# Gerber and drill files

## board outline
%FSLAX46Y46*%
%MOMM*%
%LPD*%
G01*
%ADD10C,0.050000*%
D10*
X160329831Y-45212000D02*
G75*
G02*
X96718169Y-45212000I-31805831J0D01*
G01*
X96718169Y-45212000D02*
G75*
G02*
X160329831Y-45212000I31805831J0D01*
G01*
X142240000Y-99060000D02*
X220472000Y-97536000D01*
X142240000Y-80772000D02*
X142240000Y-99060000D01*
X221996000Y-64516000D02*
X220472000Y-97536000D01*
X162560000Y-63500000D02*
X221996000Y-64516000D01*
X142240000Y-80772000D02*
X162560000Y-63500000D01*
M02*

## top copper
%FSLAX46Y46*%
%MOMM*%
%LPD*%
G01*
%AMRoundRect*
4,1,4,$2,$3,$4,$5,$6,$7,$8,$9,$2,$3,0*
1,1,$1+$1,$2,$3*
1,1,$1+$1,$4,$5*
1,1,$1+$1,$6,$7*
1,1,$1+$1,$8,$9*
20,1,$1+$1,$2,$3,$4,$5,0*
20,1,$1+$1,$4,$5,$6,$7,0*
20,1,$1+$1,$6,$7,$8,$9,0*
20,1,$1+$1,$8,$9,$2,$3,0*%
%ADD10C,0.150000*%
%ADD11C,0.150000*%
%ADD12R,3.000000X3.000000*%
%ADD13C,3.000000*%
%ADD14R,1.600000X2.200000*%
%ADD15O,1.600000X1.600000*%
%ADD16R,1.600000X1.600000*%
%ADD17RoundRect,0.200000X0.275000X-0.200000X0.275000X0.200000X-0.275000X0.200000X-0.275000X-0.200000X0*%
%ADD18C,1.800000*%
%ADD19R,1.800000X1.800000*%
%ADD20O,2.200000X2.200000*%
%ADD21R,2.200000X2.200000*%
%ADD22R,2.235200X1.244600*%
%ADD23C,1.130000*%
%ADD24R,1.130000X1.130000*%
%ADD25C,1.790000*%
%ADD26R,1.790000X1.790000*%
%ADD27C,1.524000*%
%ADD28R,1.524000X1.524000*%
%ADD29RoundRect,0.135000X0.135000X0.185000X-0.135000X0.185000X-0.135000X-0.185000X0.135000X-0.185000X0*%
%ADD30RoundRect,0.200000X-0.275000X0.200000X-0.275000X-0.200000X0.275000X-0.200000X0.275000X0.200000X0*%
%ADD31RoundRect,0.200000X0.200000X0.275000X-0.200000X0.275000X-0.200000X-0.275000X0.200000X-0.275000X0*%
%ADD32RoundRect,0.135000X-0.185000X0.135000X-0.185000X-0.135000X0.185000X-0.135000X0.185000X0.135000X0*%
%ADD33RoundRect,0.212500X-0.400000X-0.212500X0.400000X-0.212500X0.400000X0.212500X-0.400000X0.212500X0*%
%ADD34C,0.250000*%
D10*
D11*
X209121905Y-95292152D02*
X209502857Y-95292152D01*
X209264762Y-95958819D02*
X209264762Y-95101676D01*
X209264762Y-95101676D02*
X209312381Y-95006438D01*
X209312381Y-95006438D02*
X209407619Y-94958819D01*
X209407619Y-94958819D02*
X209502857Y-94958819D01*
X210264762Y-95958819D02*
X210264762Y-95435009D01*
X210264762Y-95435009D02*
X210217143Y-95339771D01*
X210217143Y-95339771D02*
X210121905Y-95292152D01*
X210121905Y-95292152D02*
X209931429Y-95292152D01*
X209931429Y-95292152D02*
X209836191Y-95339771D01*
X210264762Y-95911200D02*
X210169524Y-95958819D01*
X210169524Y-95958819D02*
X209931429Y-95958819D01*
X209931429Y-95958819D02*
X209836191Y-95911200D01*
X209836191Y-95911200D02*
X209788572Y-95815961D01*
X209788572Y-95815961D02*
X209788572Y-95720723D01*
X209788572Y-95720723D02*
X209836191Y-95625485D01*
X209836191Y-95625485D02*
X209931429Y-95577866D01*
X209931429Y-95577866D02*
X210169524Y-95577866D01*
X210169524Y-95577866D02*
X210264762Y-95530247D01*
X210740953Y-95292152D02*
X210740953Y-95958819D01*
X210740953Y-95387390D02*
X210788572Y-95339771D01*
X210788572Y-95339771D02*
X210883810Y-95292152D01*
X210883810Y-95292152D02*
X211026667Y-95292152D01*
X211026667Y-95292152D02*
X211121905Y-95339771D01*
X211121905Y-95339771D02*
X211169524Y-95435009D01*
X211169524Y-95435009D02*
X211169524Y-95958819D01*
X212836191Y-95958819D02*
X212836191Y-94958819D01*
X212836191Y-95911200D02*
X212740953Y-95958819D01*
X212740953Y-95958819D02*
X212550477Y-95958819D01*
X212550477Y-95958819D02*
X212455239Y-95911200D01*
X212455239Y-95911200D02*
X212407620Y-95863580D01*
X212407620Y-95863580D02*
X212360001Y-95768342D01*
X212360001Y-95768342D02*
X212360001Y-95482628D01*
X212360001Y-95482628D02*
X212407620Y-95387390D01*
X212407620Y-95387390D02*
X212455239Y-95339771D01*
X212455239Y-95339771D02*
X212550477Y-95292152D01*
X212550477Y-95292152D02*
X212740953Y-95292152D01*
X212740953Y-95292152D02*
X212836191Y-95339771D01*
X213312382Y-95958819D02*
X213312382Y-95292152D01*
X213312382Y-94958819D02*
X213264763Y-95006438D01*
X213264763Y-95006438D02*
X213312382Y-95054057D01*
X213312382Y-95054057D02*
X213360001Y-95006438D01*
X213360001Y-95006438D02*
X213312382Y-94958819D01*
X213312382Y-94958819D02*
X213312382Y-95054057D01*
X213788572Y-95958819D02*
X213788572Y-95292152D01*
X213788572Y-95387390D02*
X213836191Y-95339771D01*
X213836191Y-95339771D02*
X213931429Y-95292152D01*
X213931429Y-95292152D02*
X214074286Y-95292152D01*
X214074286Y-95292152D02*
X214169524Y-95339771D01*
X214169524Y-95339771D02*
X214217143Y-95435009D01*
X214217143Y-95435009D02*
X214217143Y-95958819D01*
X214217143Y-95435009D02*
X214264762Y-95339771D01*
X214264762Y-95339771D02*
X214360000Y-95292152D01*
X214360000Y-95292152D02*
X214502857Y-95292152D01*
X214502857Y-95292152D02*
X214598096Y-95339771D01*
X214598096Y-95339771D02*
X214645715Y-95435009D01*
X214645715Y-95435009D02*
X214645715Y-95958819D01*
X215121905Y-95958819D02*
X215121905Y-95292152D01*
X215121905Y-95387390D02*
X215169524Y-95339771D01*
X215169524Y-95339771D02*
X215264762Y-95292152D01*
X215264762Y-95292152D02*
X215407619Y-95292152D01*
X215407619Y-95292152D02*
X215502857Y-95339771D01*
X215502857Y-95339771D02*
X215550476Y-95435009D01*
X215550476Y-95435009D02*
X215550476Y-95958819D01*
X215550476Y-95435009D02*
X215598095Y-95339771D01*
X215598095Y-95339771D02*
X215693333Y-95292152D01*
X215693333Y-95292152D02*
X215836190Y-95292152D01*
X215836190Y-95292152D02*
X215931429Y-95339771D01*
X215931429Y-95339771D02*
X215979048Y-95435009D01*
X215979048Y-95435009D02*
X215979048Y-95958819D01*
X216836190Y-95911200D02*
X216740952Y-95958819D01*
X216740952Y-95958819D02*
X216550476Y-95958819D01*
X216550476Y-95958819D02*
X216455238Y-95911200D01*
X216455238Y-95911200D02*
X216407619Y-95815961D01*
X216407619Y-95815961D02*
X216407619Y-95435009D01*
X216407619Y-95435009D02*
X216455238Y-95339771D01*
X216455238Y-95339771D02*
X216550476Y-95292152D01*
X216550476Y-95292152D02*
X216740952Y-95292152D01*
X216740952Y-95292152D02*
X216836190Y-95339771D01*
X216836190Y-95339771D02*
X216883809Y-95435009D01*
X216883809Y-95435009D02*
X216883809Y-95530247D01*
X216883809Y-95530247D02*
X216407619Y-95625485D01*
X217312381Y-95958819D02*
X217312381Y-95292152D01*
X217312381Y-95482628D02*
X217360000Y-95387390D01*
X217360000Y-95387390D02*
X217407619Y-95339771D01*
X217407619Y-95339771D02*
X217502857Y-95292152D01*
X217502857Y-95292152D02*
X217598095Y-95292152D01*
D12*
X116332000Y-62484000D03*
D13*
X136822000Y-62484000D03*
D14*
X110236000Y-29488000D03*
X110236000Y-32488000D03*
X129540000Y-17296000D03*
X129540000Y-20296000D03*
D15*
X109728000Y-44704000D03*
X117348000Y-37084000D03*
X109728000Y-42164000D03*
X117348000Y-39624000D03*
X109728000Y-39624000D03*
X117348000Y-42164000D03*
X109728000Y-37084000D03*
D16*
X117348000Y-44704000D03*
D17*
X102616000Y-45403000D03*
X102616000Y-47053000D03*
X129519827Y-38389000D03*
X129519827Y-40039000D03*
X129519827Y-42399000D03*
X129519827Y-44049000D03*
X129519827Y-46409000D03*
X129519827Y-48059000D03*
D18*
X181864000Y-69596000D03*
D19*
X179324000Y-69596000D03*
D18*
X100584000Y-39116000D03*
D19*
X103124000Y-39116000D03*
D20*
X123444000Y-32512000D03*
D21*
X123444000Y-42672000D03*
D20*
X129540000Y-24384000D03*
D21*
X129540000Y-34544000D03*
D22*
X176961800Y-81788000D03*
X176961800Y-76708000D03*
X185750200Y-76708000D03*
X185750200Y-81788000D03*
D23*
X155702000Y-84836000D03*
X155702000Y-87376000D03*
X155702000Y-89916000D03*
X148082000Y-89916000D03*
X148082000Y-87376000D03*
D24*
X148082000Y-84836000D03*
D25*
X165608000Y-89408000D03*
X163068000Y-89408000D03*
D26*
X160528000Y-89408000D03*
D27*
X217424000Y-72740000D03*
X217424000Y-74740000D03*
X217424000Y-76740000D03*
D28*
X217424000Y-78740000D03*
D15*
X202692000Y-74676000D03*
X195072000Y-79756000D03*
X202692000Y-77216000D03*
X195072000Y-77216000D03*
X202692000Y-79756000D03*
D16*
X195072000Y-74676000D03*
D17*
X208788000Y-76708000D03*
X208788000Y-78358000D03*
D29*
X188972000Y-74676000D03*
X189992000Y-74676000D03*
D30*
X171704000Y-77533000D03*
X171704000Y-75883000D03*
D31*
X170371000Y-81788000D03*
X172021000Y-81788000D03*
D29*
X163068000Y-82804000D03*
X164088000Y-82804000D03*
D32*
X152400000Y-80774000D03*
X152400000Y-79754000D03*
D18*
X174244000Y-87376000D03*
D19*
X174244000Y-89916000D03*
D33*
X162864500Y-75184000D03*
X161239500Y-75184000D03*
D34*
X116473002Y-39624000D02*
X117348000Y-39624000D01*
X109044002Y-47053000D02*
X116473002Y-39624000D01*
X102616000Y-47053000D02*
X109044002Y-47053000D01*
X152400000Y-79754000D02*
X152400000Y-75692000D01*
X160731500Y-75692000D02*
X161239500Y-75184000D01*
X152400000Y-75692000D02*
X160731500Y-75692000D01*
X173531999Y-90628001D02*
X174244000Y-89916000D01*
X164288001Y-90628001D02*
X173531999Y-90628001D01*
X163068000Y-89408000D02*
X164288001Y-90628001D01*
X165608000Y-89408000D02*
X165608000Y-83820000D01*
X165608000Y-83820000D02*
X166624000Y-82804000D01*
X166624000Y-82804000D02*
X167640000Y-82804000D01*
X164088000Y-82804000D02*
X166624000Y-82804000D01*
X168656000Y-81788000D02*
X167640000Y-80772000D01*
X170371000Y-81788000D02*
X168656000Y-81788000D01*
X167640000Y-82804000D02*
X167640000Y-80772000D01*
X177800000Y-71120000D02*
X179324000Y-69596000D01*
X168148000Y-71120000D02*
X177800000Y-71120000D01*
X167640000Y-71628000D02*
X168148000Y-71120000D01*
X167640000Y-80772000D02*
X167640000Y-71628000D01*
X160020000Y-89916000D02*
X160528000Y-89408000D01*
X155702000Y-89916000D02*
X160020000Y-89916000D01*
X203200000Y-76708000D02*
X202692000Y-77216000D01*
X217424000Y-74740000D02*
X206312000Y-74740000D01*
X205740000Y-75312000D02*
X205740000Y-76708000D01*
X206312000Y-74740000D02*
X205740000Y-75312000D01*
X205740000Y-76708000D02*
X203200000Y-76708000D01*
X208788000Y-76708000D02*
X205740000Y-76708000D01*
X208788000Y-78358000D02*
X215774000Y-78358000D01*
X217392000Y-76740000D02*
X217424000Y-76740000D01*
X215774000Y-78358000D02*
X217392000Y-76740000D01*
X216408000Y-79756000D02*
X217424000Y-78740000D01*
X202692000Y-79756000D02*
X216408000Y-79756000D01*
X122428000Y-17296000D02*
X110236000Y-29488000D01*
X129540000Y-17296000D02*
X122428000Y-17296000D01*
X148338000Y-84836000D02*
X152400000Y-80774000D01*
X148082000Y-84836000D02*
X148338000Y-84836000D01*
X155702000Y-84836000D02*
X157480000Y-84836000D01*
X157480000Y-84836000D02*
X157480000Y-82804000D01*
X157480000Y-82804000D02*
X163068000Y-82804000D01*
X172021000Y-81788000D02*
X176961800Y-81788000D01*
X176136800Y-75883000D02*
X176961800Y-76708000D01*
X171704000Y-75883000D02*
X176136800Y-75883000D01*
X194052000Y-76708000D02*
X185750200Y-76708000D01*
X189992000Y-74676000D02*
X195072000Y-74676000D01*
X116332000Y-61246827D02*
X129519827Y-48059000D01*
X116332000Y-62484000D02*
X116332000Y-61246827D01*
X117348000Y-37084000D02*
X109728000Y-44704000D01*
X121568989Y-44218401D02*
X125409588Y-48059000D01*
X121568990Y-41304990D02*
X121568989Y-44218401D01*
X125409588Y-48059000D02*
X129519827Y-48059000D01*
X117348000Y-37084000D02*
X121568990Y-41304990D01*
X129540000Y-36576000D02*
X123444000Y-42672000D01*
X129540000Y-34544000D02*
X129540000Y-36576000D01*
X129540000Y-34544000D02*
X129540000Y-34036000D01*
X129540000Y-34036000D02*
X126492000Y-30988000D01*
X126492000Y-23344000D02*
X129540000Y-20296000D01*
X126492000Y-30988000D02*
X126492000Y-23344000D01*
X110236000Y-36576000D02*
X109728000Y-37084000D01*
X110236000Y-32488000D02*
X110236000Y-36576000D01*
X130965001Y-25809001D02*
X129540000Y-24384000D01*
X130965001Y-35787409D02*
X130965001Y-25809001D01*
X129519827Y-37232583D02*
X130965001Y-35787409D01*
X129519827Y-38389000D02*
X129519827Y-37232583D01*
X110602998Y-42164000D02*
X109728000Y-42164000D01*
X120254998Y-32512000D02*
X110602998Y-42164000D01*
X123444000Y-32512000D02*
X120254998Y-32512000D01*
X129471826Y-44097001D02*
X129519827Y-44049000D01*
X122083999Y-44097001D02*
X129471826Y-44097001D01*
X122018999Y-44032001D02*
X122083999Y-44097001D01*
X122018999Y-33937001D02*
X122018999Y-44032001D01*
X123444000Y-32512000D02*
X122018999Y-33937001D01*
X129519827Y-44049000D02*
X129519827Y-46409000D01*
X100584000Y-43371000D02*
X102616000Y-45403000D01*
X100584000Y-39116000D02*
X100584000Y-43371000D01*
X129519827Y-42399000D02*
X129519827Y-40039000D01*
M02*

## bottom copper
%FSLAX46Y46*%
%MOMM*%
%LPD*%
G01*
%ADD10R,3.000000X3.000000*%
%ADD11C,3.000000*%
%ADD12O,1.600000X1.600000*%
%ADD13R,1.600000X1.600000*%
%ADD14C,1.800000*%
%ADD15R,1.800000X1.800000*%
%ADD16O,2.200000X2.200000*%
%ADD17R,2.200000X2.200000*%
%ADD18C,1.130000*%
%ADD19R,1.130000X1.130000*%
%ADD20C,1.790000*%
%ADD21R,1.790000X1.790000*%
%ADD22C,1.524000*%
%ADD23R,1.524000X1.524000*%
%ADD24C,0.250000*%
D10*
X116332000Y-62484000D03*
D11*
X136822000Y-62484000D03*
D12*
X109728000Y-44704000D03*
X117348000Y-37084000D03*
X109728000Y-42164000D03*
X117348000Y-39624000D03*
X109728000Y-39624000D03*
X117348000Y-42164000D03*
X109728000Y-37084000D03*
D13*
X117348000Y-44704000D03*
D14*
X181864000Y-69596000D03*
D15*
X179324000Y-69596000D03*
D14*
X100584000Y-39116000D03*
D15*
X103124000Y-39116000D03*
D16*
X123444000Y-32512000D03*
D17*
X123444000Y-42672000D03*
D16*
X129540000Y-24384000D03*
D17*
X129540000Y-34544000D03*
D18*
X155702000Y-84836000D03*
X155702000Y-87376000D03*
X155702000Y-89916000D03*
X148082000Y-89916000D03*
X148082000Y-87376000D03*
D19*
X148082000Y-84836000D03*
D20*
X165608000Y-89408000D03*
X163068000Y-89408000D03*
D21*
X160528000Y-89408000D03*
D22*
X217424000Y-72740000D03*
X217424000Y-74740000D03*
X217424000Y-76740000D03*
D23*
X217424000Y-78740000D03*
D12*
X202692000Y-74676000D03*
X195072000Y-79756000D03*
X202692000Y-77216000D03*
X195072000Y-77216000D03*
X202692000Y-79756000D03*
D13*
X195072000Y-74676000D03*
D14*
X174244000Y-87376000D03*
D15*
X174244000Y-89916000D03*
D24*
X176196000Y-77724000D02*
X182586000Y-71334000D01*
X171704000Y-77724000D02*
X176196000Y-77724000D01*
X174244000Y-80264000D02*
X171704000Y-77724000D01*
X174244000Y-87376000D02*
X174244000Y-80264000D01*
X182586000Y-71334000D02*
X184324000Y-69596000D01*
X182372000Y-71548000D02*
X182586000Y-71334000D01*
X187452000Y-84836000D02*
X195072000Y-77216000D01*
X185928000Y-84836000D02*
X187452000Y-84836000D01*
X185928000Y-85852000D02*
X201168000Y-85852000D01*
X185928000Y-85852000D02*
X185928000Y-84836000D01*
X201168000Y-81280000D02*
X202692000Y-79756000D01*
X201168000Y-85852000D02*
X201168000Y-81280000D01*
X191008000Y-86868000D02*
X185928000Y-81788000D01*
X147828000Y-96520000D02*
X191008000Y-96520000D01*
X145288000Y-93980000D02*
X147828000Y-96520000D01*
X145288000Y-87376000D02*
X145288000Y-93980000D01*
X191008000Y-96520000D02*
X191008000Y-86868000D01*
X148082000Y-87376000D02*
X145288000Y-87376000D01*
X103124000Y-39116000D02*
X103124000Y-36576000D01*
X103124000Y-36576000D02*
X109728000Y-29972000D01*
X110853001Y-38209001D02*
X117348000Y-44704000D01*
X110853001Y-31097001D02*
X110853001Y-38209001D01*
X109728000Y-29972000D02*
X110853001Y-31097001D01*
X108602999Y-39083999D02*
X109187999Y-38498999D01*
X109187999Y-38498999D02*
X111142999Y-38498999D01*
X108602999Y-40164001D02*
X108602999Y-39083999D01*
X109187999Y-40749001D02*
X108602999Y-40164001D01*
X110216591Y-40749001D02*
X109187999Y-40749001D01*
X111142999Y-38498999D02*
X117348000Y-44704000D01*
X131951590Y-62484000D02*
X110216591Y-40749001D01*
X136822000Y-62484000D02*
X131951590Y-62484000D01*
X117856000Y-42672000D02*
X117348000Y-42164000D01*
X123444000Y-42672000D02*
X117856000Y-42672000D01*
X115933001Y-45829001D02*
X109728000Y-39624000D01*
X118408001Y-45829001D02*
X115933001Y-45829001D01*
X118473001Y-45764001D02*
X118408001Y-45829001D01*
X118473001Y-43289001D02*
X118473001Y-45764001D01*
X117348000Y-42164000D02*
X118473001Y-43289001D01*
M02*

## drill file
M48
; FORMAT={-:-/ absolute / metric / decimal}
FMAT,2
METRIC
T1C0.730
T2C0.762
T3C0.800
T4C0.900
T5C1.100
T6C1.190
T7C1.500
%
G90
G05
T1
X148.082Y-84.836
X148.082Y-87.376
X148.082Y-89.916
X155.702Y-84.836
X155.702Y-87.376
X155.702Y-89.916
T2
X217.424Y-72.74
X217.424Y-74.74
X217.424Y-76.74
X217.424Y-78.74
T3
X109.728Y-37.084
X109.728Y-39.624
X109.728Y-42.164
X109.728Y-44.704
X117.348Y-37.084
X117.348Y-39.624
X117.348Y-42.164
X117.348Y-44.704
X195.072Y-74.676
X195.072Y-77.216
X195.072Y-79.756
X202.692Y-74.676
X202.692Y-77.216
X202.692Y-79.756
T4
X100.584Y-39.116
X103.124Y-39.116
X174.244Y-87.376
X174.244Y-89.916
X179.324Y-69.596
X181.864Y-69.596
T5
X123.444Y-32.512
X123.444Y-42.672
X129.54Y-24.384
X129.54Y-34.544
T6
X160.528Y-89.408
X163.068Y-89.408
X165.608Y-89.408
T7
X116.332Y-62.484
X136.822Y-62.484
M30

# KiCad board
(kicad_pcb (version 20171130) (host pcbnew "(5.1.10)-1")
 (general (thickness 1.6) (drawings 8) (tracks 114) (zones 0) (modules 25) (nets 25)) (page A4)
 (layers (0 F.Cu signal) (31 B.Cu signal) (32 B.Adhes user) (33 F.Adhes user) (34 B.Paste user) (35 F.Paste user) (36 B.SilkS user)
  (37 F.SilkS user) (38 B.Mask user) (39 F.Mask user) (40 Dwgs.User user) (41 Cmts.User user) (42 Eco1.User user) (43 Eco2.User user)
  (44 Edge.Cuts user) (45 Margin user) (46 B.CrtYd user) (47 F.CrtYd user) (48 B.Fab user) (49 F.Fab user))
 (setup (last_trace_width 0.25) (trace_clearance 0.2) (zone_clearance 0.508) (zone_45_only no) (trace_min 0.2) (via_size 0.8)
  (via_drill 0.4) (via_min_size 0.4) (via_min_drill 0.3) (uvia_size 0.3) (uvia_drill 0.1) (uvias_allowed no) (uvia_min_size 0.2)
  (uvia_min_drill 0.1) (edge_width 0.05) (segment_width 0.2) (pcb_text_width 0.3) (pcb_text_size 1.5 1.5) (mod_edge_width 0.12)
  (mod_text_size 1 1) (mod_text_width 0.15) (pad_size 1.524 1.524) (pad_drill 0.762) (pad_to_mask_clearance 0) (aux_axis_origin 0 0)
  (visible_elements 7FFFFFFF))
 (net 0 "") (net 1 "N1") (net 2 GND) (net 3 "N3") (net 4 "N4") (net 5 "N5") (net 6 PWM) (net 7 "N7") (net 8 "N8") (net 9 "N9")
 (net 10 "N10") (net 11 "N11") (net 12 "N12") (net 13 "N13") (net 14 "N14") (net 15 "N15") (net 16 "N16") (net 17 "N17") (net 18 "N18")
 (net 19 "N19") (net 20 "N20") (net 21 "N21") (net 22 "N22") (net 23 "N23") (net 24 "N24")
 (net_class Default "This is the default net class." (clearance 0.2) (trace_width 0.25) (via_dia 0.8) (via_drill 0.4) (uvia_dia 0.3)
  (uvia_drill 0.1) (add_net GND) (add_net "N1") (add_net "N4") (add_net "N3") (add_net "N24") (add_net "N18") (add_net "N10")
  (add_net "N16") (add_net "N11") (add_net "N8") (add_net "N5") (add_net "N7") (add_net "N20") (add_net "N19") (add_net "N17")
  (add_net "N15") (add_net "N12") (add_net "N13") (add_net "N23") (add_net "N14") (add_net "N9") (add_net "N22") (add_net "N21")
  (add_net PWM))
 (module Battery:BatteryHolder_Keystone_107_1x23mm (layer F.Cu) (at 116.332 62.484)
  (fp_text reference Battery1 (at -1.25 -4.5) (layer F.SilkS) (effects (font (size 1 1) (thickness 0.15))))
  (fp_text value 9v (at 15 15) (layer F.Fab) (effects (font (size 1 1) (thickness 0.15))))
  (pad 1 thru_hole rect (at 0 0) (size 3 3) (drill 1.5) (layers *.Cu *.Mask) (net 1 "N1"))
  (pad 2 thru_hole circle (at 20.49 0) (size 3 3) (drill 1.5) (layers *.Cu *.Mask) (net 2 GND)))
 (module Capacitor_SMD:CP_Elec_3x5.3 (layer F.Cu) (at 110.236 30.988 90)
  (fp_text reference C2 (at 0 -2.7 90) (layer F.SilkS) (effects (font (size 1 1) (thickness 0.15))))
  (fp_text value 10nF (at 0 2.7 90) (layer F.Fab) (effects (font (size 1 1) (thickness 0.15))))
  (pad 2 smd rect (at 1.5 0 90) (size 2.2 1.6) (layers F.Cu F.Paste F.Mask) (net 2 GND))
  (pad 1 smd rect (at -1.5 0 90) (size 2.2 1.6) (layers F.Cu F.Paste F.Mask) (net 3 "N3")))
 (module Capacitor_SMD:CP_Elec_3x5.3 (layer F.Cu) (at 129.54 18.796 90)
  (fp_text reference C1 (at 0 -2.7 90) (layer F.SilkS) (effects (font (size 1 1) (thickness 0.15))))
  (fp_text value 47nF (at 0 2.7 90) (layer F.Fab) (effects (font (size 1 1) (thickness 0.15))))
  (pad 2 smd rect (at 1.5 0 90) (size 2.2 1.6) (layers F.Cu F.Paste F.Mask) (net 2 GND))
  (pad 1 smd rect (at -1.5 0 90) (size 2.2 1.6) (layers F.Cu F.Paste F.Mask) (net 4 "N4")))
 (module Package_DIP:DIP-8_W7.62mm (layer F.Cu) (at 117.348 44.704 180)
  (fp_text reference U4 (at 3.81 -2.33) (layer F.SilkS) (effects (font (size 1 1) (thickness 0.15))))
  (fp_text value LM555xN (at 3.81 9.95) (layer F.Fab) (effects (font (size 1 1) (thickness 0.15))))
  (pad 8 thru_hole oval (at 7.62 0 180) (size 1.6 1.6) (drill 0.8) (layers *.Cu *.Mask) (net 1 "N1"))
  (pad 4 thru_hole oval (at 0 7.62 180) (size 1.6 1.6) (drill 0.8) (layers *.Cu *.Mask) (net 1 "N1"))
  (pad 7 thru_hole oval (at 7.62 2.54 180) (size 1.6 1.6) (drill 0.8) (layers *.Cu *.Mask) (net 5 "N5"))
  (pad 3 thru_hole oval (at 0 5.08 180) (size 1.6 1.6) (drill 0.8) (layers *.Cu *.Mask) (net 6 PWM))
  (pad 6 thru_hole oval (at 7.62 5.08 180) (size 1.6 1.6) (drill 0.8) (layers *.Cu *.Mask) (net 4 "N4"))
  (pad 2 thru_hole oval (at 0 2.54 180) (size 1.6 1.6) (drill 0.8) (layers *.Cu *.Mask) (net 4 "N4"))
  (pad 5 thru_hole oval (at 7.62 7.62 180) (size 1.6 1.6) (drill 0.8) (layers *.Cu *.Mask) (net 3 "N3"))
  (pad 1 thru_hole rect (at 0 0 180) (size 1.6 1.6) (drill 0.8) (layers *.Cu *.Mask) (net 2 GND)))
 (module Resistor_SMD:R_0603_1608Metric (layer F.Cu) (at 102.616 46.228 90)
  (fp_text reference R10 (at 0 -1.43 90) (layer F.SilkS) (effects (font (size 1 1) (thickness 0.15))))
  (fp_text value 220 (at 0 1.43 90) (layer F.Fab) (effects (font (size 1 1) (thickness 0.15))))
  (pad 2 smd roundrect (at 0.825 0 90) (size 0.8 0.95) (layers F.Cu F.Paste F.Mask) (roundrect_rratio 0.25) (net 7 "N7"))
  (pad 1 smd roundrect (at -0.825 0 90) (size 0.8 0.95) (layers F.Cu F.Paste F.Mask) (roundrect_rratio 0.25) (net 6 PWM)))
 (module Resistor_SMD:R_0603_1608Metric (layer F.Cu) (at 129.519827 39.214 90)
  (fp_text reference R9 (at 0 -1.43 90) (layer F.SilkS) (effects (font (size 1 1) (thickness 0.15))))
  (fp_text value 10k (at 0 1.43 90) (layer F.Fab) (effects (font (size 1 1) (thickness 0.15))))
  (pad 2 smd roundrect (at 0.825 0 90) (size 0.8 0.95) (layers F.Cu F.Paste F.Mask) (roundrect_rratio 0.25) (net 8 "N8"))
  (pad 1 smd roundrect (at -0.825 0 90) (size 0.8 0.95) (layers F.Cu F.Paste F.Mask) (roundrect_rratio 0.25) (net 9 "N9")))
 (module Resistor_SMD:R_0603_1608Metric (layer F.Cu) (at 129.519827 43.224 90)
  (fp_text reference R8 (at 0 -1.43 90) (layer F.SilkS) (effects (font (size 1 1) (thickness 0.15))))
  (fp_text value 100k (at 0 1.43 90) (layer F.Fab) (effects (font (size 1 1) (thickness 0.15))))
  (pad 2 smd roundrect (at 0.825 0 90) (size 0.8 0.95) (layers F.Cu F.Paste F.Mask) (roundrect_rratio 0.25) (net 9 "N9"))
  (pad 1 smd roundrect (at -0.825 0 90) (size 0.8 0.95) (layers F.Cu F.Paste F.Mask) (roundrect_rratio 0.25) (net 5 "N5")))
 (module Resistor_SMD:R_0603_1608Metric (layer F.Cu) (at 129.519827 47.234 90)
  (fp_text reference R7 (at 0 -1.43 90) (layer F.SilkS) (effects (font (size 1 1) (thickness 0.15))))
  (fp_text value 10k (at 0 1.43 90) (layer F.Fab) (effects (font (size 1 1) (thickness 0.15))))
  (pad 2 smd roundrect (at 0.825 0 90) (size 0.8 0.95) (layers F.Cu F.Paste F.Mask) (roundrect_rratio 0.25) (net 5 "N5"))
  (pad 1 smd roundrect (at -0.825 0 90) (size 0.8 0.95) (layers F.Cu F.Paste F.Mask) (roundrect_rratio 0.25) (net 1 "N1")))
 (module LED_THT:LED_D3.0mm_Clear (layer F.Cu) (at 179.324 69.596)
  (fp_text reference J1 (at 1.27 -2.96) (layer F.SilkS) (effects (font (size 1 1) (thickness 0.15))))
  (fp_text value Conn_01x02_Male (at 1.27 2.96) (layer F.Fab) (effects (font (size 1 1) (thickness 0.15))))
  (pad 2 thru_hole circle (at 2.54 0) (size 1.8 1.8) (drill 0.9) (layers *.Cu *.Mask) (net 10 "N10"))
  (pad 1 thru_hole rect (at 0 0) (size 1.8 1.8) (drill 0.9) (layers *.Cu *.Mask) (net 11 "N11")))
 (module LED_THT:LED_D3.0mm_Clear (layer F.Cu) (at 103.124 39.116 180)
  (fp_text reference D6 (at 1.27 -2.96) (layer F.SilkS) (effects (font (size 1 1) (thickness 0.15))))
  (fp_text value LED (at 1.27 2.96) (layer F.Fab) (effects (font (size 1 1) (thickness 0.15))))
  (pad 2 thru_hole circle (at 2.54 0 180) (size 1.8 1.8) (drill 0.9) (layers *.Cu *.Mask) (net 7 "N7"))
  (pad 1 thru_hole rect (at 0 0 180) (size 1.8 1.8) (drill 0.9) (layers *.Cu *.Mask) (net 2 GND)))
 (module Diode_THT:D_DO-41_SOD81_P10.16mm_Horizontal (layer F.Cu) (at 123.444 42.672 90)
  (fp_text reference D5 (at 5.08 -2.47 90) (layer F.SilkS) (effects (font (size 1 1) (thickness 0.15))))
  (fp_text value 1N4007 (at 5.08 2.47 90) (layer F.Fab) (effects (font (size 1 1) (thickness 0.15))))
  (pad 2 thru_hole oval (at 10.16 0 90) (size 2.2 2.2) (drill 1.1) (layers *.Cu *.Mask) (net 5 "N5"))
  (pad 1 thru_hole rect (at 0 0 90) (size 2.2 2.2) (drill 1.1) (layers *.Cu *.Mask) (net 4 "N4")))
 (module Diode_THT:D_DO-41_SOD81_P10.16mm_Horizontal (layer F.Cu) (at 129.54 34.544 90)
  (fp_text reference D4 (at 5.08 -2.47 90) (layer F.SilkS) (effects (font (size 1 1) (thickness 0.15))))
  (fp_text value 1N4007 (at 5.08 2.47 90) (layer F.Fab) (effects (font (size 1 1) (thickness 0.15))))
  (pad 2 thru_hole oval (at 10.16 0 90) (size 2.2 2.2) (drill 1.1) (layers *.Cu *.Mask) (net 8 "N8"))
  (pad 1 thru_hole rect (at 0 0 90) (size 2.2 2.2) (drill 1.1) (layers *.Cu *.Mask) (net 4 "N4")))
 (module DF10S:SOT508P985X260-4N (layer F.Cu) (at 181.356 79.248 180)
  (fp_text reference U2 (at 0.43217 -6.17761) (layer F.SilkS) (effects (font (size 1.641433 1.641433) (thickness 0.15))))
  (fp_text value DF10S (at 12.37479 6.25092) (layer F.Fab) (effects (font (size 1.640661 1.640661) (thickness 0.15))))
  (pad 4 smd rect (at 4.3942 -2.54 180) (size 2.2352 1.2446) (layers F.Cu F.Paste F.Mask) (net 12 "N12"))
  (pad 3 smd rect (at 4.3942 2.54 180) (size 2.2352 1.2446) (layers F.Cu F.Paste F.Mask) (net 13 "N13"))
  (pad 2 smd rect (at -4.3942 2.54 180) (size 2.2352 1.2446) (layers F.Cu F.Paste F.Mask) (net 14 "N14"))
  (pad 1 smd rect (at -4.3942 -2.54 180) (size 2.2352 1.2446) (layers F.Cu F.Paste F.Mask) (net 2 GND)))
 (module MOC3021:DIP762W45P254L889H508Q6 (layer F.Cu) (at 151.892 87.376)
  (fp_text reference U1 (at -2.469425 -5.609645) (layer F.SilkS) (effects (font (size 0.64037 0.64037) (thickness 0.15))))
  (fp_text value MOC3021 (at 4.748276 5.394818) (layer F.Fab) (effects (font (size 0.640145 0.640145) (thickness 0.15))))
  (pad 6 thru_hole circle (at 3.81 -2.54) (size 1.13 1.13) (drill 0.73) (layers *.Cu *.Mask) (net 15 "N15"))
  (pad 5 thru_hole circle (at 3.81 0) (size 1.13 1.13) (drill 0.73) (layers *.Cu *.Mask))
  (pad 4 thru_hole circle (at 3.81 2.54) (size 1.13 1.13) (drill 0.73) (layers *.Cu *.Mask) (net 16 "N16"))
  (pad 3 thru_hole circle (at -3.81 2.54) (size 1.13 1.13) (drill 0.73) (layers *.Cu *.Mask))
  (pad 2 thru_hole circle (at -3.81 0) (size 1.13 1.13) (drill 0.73) (layers *.Cu *.Mask) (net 2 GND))
  (pad 1 thru_hole rect (at -3.81 -2.54) (size 1.13 1.13) (drill 0.73) (layers *.Cu *.Mask) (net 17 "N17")))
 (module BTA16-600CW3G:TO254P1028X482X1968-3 (layer F.Cu) (at 160.528 89.408)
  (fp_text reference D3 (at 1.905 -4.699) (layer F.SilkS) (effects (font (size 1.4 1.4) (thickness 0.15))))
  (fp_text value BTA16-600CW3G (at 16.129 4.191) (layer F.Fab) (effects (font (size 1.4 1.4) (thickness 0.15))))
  (pad 3 thru_hole circle (at 5.08 0) (size 1.79 1.79) (drill 1.19) (layers *.Cu *.Mask) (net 11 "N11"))
  (pad 2 thru_hole circle (at 2.54 0) (size 1.79 1.79) (drill 1.19) (layers *.Cu *.Mask) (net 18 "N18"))
  (pad 1 thru_hole rect (at 0 0) (size 1.79 1.79) (drill 1.19) (layers *.Cu *.Mask) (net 16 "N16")))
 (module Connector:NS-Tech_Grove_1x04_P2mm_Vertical (layer F.Cu) (at 217.424 78.74 180)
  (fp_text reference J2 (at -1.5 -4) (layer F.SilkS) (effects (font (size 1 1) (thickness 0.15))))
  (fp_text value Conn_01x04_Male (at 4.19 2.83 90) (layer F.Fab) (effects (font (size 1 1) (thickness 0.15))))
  (pad 4 thru_hole circle (at 0 6 180) (size 1.524 1.524) (drill 0.762) (layers *.Cu *.Mask) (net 6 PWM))
  (pad 3 thru_hole circle (at 0 4 180) (size 1.524 1.524) (drill 0.762) (layers *.Cu *.Mask) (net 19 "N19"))
  (pad 2 thru_hole circle (at 0 2 180) (size 1.524 1.524) (drill 0.762) (layers *.Cu *.Mask) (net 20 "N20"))
  (pad 1 thru_hole rect (at 0 0 180) (size 1.524 1.524) (drill 0.762) (layers *.Cu *.Mask) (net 2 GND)))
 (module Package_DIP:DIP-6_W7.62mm (layer F.Cu) (at 195.072 74.676)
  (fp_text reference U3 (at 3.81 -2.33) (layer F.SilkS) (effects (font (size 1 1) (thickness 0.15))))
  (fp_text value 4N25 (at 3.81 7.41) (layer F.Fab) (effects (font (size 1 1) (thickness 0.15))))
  (pad 6 thru_hole oval (at 7.62 0) (size 1.6 1.6) (drill 0.8) (layers *.Cu *.Mask) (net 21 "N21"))
  (pad 3 thru_hole oval (at 0 5.08) (size 1.6 1.6) (drill 0.8) (layers *.Cu *.Mask) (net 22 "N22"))
  (pad 5 thru_hole oval (at 7.62 2.54) (size 1.6 1.6) (drill 0.8) (layers *.Cu *.Mask) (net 19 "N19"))
  (pad 2 thru_hole oval (at 0 2.54) (size 1.6 1.6) (drill 0.8) (layers *.Cu *.Mask) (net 2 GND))
  (pad 4 thru_hole oval (at 7.62 5.08) (size 1.6 1.6) (drill 0.8) (layers *.Cu *.Mask) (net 2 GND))
  (pad 1 thru_hole rect (at 0 0) (size 1.6 1.6) (drill 0.8) (layers *.Cu *.Mask) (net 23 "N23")))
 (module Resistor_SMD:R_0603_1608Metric (layer F.Cu) (at 208.788 77.533 90)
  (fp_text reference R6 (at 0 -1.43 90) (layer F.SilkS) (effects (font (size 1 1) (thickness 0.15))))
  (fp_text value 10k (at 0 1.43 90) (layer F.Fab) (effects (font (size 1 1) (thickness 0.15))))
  (pad 2 smd roundrect (at 0.825 0 90) (size 0.8 0.95) (layers F.Cu F.Paste F.Mask) (roundrect_rratio 0.25) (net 19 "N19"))
  (pad 1 smd roundrect (at -0.825 0 90) (size 0.8 0.95) (layers F.Cu F.Paste F.Mask) (roundrect_rratio 0.25) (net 20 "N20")))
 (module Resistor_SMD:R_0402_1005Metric (layer F.Cu) (at 189.482 74.676 180)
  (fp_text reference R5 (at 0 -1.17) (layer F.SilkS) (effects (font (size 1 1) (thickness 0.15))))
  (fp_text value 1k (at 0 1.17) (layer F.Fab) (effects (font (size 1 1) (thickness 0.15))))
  (pad 2 smd roundrect (at 0.51 0 180) (size 0.54 0.64) (layers F.Cu F.Paste F.Mask) (roundrect_rratio 0.25) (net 14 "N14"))
  (pad 1 smd roundrect (at -0.51 0 180) (size 0.54 0.64) (layers F.Cu F.Paste F.Mask) (roundrect_rratio 0.25) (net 23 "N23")))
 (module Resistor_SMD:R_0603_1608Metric (layer F.Cu) (at 171.704 76.708 270)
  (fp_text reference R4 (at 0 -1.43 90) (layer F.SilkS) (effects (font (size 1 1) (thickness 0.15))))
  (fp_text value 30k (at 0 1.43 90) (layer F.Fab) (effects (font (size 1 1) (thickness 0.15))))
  (pad 2 smd roundrect (at 0.825 0 270) (size 0.8 0.95) (layers F.Cu F.Paste F.Mask) (roundrect_rratio 0.25) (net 10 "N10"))
  (pad 1 smd roundrect (at -0.825 0 270) (size 0.8 0.95) (layers F.Cu F.Paste F.Mask) (roundrect_rratio 0.25) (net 13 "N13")))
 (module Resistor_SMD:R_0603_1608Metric (layer F.Cu) (at 171.196 81.788 180)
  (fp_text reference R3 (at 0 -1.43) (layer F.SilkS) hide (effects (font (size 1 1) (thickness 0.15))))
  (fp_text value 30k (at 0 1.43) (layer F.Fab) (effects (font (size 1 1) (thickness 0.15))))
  (pad 2 smd roundrect (at 0.825 0 180) (size 0.8 0.95) (layers F.Cu F.Paste F.Mask) (roundrect_rratio 0.25) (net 11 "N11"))
  (pad 1 smd roundrect (at -0.825 0 180) (size 0.8 0.95) (layers F.Cu F.Paste F.Mask) (roundrect_rratio 0.25) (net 12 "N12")))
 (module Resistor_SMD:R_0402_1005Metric (layer F.Cu) (at 163.578 82.804 180)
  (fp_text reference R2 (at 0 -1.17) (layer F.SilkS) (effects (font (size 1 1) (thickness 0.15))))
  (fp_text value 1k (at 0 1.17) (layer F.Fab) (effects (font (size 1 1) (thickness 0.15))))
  (pad 2 smd roundrect (at 0.51 0 180) (size 0.54 0.64) (layers F.Cu F.Paste F.Mask) (roundrect_rratio 0.25) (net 15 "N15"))
  (pad 1 smd roundrect (at -0.51 0 180) (size 0.54 0.64) (layers F.Cu F.Paste F.Mask) (roundrect_rratio 0.25) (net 11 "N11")))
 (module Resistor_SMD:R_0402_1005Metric (layer F.Cu) (at 152.4 80.264 270)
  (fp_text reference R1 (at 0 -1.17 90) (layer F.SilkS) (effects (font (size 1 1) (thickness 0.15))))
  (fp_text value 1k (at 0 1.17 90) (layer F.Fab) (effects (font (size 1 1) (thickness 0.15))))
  (pad 2 smd roundrect (at 0.51 0 270) (size 0.54 0.64) (layers F.Cu F.Paste F.Mask) (roundrect_rratio 0.25) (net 17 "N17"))
  (pad 1 smd roundrect (at -0.51 0 270) (size 0.54 0.64) (layers F.Cu F.Paste F.Mask) (roundrect_rratio 0.25) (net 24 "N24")))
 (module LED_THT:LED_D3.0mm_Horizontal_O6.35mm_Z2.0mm (layer F.Cu) (at 174.244 89.916 90)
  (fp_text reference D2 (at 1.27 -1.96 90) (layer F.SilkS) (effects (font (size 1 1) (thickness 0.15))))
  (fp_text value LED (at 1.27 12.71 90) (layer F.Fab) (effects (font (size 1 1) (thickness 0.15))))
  (pad 2 thru_hole circle (at 2.54 0 90) (size 1.8 1.8) (drill 0.9) (layers *.Cu *.Mask) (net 10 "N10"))
  (pad 1 thru_hole rect (at 0 0 90) (size 1.8 1.8) (drill 0.9) (layers *.Cu *.Mask) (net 18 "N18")))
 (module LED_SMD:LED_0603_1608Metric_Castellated (layer F.Cu) (at 162.052 75.184)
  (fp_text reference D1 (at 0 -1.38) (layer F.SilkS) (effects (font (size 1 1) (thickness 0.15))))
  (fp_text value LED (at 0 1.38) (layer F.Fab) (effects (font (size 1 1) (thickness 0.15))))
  (pad 2 smd roundrect (at 0.8125 0) (size 1.225 0.85) (layers F.Cu F.Paste F.Mask) (roundrect_rratio 0.25) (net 6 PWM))
  (pad 1 smd roundrect (at -0.8125 0) (size 1.225 0.85) (layers F.Cu F.Paste F.Mask) (roundrect_rratio 0.25) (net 24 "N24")))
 (gr_circle (center 128.524 45.212) (end 114.3 16.764) (layer Edge.Cuts) (width 0.05))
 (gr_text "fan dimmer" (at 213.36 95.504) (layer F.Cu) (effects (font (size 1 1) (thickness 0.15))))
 (gr_line (start 142.24 99.06) (end 220.472 97.536) (layer Edge.Cuts) (width 0.05))
 (gr_line (start 142.24 80.772) (end 142.24 99.06) (layer Edge.Cuts) (width 0.05))
 (gr_line (start 221.996 64.516) (end 220.472 97.536) (layer Edge.Cuts) (width 0.05))
 (gr_line (start 162.56 63.5) (end 221.996 64.516) (layer Edge.Cuts) (width 0.05))
 (gr_line (start 142.24 80.772) (end 162.56 63.5) (layer Edge.Cuts) (width 0.05))
 (segment (start 116.473002 39.624) (end 117.348 39.624) (width 0.25) (layer F.Cu) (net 6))
 (segment (start 109.044002 47.053) (end 116.473002 39.624) (width 0.25) (layer F.Cu) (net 6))
 (segment (start 102.616 47.053) (end 109.044002 47.053) (width 0.25) (layer F.Cu) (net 6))
 (segment (start 152.4 79.754) (end 152.4 75.692) (width 0.25) (layer F.Cu) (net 24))
 (segment (start 160.7315 75.692) (end 161.2395 75.184) (width 0.25) (layer F.Cu) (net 24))
 (segment (start 152.4 75.692) (end 160.7315 75.692) (width 0.25) (layer F.Cu) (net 24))
 (segment (start 176.196 77.724) (end 182.586 71.334) (width 0.25) (layer B.Cu) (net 10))
 (segment (start 171.704 77.724) (end 176.196 77.724) (width 0.25) (layer B.Cu) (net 10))
 (segment (start 174.244 80.264) (end 171.704 77.724) (width 0.25) (layer B.Cu) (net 10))
 (segment (start 174.244 87.376) (end 174.244 80.264) (width 0.25) (layer B.Cu) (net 10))
 (segment (start 182.586 71.334) (end 184.324 69.596) (width 0.25) (layer B.Cu) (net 10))
 (segment (start 182.372 71.548) (end 182.586 71.334) (width 0.25) (layer B.Cu) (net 10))
 (segment (start 173.531999 90.628001) (end 174.244 89.916) (width 0.25) (layer F.Cu) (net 18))
 (segment (start 164.288001 90.628001) (end 173.531999 90.628001) (width 0.25) (layer F.Cu) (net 18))
 (segment (start 163.068 89.408) (end 164.288001 90.628001) (width 0.25) (layer F.Cu) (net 18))
 (segment (start 165.608 89.408) (end 165.608 83.82) (width 0.25) (layer F.Cu) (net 11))
 (segment (start 165.608 83.82) (end 166.624 82.804) (width 0.25) (layer F.Cu) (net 11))
 (segment (start 166.624 82.804) (end 167.64 82.804) (width 0.25) (layer F.Cu) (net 11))
 (segment (start 164.088 82.804) (end 166.624 82.804) (width 0.25) (layer F.Cu) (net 11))
 (segment (start 168.656 81.788) (end 167.64 80.772) (width 0.25) (layer F.Cu) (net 11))
 (segment (start 170.371 81.788) (end 168.656 81.788) (width 0.25) (layer F.Cu) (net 11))
 (segment (start 167.64 82.804) (end 167.64 80.772) (width 0.25) (layer F.Cu) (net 11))
 (segment (start 177.8 71.12) (end 179.324 69.596) (width 0.25) (layer F.Cu) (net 11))
 (segment (start 168.148 71.12) (end 177.8 71.12) (width 0.25) (layer F.Cu) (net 11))
 (segment (start 167.64 71.628) (end 168.148 71.12) (width 0.25) (layer F.Cu) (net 11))
 (segment (start 167.64 80.772) (end 167.64 71.628) (width 0.25) (layer F.Cu) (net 11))
 (segment (start 160.02 89.916) (end 160.528 89.408) (width 0.25) (layer F.Cu) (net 16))
 (segment (start 155.702 89.916) (end 160.02 89.916) (width 0.25) (layer F.Cu) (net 16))
 (segment (start 203.2 76.708) (end 202.692 77.216) (width 0.25) (layer F.Cu) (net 19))
 (segment (start 217.424 74.74) (end 206.312 74.74) (width 0.25) (layer F.Cu) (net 19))
 (segment (start 205.74 75.312) (end 205.74 76.708) (width 0.25) (layer F.Cu) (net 19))
 (segment (start 206.312 74.74) (end 205.74 75.312) (width 0.25) (layer F.Cu) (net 19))
 (segment (start 205.74 76.708) (end 203.2 76.708) (width 0.25) (layer F.Cu) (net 19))
 (segment (start 208.788 76.708) (end 205.74 76.708) (width 0.25) (layer F.Cu) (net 19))
 (segment (start 208.788 78.358) (end 215.774 78.358) (width 0.25) (layer F.Cu) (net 20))
 (segment (start 217.392 76.74) (end 217.424 76.74) (width 0.25) (layer F.Cu) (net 20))
 (segment (start 215.774 78.358) (end 217.392 76.74) (width 0.25) (layer F.Cu) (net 20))
 (segment (start 216.408 79.756) (end 217.424 78.74) (width 0.25) (layer F.Cu) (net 2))
 (segment (start 202.692 79.756) (end 216.408 79.756) (width 0.25) (layer F.Cu) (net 2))
 (segment (start 187.452 84.836) (end 195.072 77.216) (width 0.25) (layer B.Cu) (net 2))
 (segment (start 185.928 84.836) (end 187.452 84.836) (width 0.25) (layer B.Cu) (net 2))
 (segment (start 185.928 85.852) (end 201.168 85.852) (width 0.25) (layer B.Cu) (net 2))
 (segment (start 185.928 85.852) (end 185.928 84.836) (width 0.25) (layer B.Cu) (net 2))
 (segment (start 201.168 81.28) (end 202.692 79.756) (width 0.25) (layer B.Cu) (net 2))
 (segment (start 201.168 85.852) (end 201.168 81.28) (width 0.25) (layer B.Cu) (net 2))
 (segment (start 191.008 86.868) (end 185.928 81.788) (width 0.25) (layer B.Cu) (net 2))
 (segment (start 147.828 96.52) (end 191.008 96.52) (width 0.25) (layer B.Cu) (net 2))
 (segment (start 145.288 93.98) (end 147.828 96.52) (width 0.25) (layer B.Cu) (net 2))
 (segment (start 145.288 87.376) (end 145.288 93.98) (width 0.25) (layer B.Cu) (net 2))
 (segment (start 191.008 96.52) (end 191.008 86.868) (width 0.25) (layer B.Cu) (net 2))
 (segment (start 148.082 87.376) (end 145.288 87.376) (width 0.25) (layer B.Cu) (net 2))
 (segment (start 103.124 39.116) (end 103.124 36.576) (width 0.25) (layer B.Cu) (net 2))
 (segment (start 103.124 36.576) (end 109.728 29.972) (width 0.25) (layer B.Cu) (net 2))
 (segment (start 110.853001 38.209001) (end 117.348 44.704) (width 0.25) (layer B.Cu) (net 2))
 (segment (start 110.853001 31.097001) (end 110.853001 38.209001) (width 0.25) (layer B.Cu) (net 2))
 (segment (start 109.728 29.972) (end 110.853001 31.097001) (width 0.25) (layer B.Cu) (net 2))
 (segment (start 122.428 17.296) (end 110.236 29.488) (width 0.25) (layer F.Cu) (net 2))
 (segment (start 129.54 17.296) (end 122.428 17.296) (width 0.25) (layer F.Cu) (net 2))
 (segment (start 108.602999 39.083999) (end 109.187999 38.498999) (width 0.25) (layer B.Cu) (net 2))
 (segment (start 109.187999 38.498999) (end 111.142999 38.498999) (width 0.25) (layer B.Cu) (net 2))
 (segment (start 108.602999 40.164001) (end 108.602999 39.083999) (width 0.25) (layer B.Cu) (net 2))
 (segment (start 109.187999 40.749001) (end 108.602999 40.164001) (width 0.25) (layer B.Cu) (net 2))
 (segment (start 110.216591 40.749001) (end 109.187999 40.749001) (width 0.25) (layer B.Cu) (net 2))
 (segment (start 111.142999 38.498999) (end 117.348 44.704) (width 0.25) (layer B.Cu) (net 2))
 (segment (start 131.95159 62.484) (end 110.216591 40.749001) (width 0.25) (layer B.Cu) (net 2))
 (segment (start 136.822 62.484) (end 131.95159 62.484) (width 0.25) (layer B.Cu) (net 2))
 (segment (start 148.338 84.836) (end 152.4 80.774) (width 0.25) (layer F.Cu) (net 17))
 (segment (start 148.082 84.836) (end 148.338 84.836) (width 0.25) (layer F.Cu) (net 17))
 (segment (start 155.702 84.836) (end 157.48 84.836) (width 0.25) (layer F.Cu) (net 15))
 (segment (start 157.48 84.836) (end 157.48 82.804) (width 0.25) (layer F.Cu) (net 15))
 (segment (start 157.48 82.804) (end 163.068 82.804) (width 0.25) (layer F.Cu) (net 15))
 (segment (start 172.021 81.788) (end 176.9618 81.788) (width 0.25) (layer F.Cu) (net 12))
 (segment (start 176.1368 75.883) (end 176.9618 76.708) (width 0.25) (layer F.Cu) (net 13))
 (segment (start 171.704 75.883) (end 176.1368 75.883) (width 0.25) (layer F.Cu) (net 13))
 (segment (start 194.052 76.708) (end 185.7502 76.708) (width 0.25) (layer F.Cu) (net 14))
 (segment (start 189.992 74.676) (end 195.072 74.676) (width 0.25) (layer F.Cu) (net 23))
 (segment (start 116.332 61.246827) (end 129.519827 48.059) (width 0.25) (layer F.Cu) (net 1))
 (segment (start 116.332 62.484) (end 116.332 61.246827) (width 0.25) (layer F.Cu) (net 1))
 (segment (start 117.348 37.084) (end 109.728 44.704) (width 0.25) (layer F.Cu) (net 1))
 (segment (start 121.568989 44.218401) (end 125.409588 48.059) (width 0.25) (layer F.Cu) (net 1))
 (segment (start 121.56899 41.30499) (end 121.568989 44.218401) (width 0.25) (layer F.Cu) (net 1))
 (segment (start 125.409588 48.059) (end 129.519827 48.059) (width 0.25) (layer F.Cu) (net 1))
 (segment (start 117.348 37.084) (end 121.56899 41.30499) (width 0.25) (layer F.Cu) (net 1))
 (segment (start 117.856 42.672) (end 117.348 42.164) (width 0.25) (layer B.Cu) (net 4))
 (segment (start 123.444 42.672) (end 117.856 42.672) (width 0.25) (layer B.Cu) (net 4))
 (segment (start 115.933001 45.829001) (end 109.728 39.624) (width 0.25) (layer B.Cu) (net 4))
 (segment (start 118.408001 45.829001) (end 115.933001 45.829001) (width 0.25) (layer B.Cu) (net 4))
 (segment (start 118.473001 45.764001) (end 118.408001 45.829001) (width 0.25) (layer B.Cu) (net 4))
 (segment (start 118.473001 43.289001) (end 118.473001 45.764001) (width 0.25) (layer B.Cu) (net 4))
 (segment (start 117.348 42.164) (end 118.473001 43.289001) (width 0.25) (layer B.Cu) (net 4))
 (segment (start 129.54 36.576) (end 123.444 42.672) (width 0.25) (layer F.Cu) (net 4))
 (segment (start 129.54 34.544) (end 129.54 36.576) (width 0.25) (layer F.Cu) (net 4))
 (segment (start 129.54 34.544) (end 129.54 34.036) (width 0.25) (layer F.Cu) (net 4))
 (segment (start 129.54 34.036) (end 126.492 30.988) (width 0.25) (layer F.Cu) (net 4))
 (segment (start 126.492 23.344) (end 129.54 20.296) (width 0.25) (layer F.Cu) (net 4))
 (segment (start 126.492 30.988) (end 126.492 23.344) (width 0.25) (layer F.Cu) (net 4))
 (segment (start 110.236 36.576) (end 109.728 37.084) (width 0.25) (layer F.Cu) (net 3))
 (segment (start 110.236 32.488) (end 110.236 36.576) (width 0.25) (layer F.Cu) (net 3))
 (segment (start 130.965001 25.809001) (end 129.54 24.384) (width 0.25) (layer F.Cu) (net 8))
 (segment (start 130.965001 35.787409) (end 130.965001 25.809001) (width 0.25) (layer F.Cu) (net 8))
 (segment (start 129.519827 37.232583) (end 130.965001 35.787409) (width 0.25) (layer F.Cu) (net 8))
 (segment (start 129.519827 38.389) (end 129.519827 37.232583) (width 0.25) (layer F.Cu) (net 8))
 (segment (start 110.602998 42.164) (end 109.728 42.164) (width 0.25) (layer F.Cu) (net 5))
 (segment (start 120.254998 32.512) (end 110.602998 42.164) (width 0.25) (layer F.Cu) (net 5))
 (segment (start 123.444 32.512) (end 120.254998 32.512) (width 0.25) (layer F.Cu) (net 5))
 (segment (start 129.471826 44.097001) (end 129.519827 44.049) (width 0.25) (layer F.Cu) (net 5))
 (segment (start 122.083999 44.097001) (end 129.471826 44.097001) (width 0.25) (layer F.Cu) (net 5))
 (segment (start 122.018999 44.032001) (end 122.083999 44.097001) (width 0.25) (layer F.Cu) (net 5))
 (segment (start 122.018999 33.937001) (end 122.018999 44.032001) (width 0.25) (layer F.Cu) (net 5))
 (segment (start 123.444 32.512) (end 122.018999 33.937001) (width 0.25) (layer F.Cu) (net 5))
 (segment (start 129.519827 44.049) (end 129.519827 46.409) (width 0.25) (layer F.Cu) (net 5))
 (segment (start 100.584 43.371) (end 102.616 45.403) (width 0.25) (layer F.Cu) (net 7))
 (segment (start 100.584 39.116) (end 100.584 43.371) (width 0.25) (layer F.Cu) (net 7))
 (segment (start 129.519827 42.399) (end 129.519827 40.039) (width 0.25) (layer F.Cu) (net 9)))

